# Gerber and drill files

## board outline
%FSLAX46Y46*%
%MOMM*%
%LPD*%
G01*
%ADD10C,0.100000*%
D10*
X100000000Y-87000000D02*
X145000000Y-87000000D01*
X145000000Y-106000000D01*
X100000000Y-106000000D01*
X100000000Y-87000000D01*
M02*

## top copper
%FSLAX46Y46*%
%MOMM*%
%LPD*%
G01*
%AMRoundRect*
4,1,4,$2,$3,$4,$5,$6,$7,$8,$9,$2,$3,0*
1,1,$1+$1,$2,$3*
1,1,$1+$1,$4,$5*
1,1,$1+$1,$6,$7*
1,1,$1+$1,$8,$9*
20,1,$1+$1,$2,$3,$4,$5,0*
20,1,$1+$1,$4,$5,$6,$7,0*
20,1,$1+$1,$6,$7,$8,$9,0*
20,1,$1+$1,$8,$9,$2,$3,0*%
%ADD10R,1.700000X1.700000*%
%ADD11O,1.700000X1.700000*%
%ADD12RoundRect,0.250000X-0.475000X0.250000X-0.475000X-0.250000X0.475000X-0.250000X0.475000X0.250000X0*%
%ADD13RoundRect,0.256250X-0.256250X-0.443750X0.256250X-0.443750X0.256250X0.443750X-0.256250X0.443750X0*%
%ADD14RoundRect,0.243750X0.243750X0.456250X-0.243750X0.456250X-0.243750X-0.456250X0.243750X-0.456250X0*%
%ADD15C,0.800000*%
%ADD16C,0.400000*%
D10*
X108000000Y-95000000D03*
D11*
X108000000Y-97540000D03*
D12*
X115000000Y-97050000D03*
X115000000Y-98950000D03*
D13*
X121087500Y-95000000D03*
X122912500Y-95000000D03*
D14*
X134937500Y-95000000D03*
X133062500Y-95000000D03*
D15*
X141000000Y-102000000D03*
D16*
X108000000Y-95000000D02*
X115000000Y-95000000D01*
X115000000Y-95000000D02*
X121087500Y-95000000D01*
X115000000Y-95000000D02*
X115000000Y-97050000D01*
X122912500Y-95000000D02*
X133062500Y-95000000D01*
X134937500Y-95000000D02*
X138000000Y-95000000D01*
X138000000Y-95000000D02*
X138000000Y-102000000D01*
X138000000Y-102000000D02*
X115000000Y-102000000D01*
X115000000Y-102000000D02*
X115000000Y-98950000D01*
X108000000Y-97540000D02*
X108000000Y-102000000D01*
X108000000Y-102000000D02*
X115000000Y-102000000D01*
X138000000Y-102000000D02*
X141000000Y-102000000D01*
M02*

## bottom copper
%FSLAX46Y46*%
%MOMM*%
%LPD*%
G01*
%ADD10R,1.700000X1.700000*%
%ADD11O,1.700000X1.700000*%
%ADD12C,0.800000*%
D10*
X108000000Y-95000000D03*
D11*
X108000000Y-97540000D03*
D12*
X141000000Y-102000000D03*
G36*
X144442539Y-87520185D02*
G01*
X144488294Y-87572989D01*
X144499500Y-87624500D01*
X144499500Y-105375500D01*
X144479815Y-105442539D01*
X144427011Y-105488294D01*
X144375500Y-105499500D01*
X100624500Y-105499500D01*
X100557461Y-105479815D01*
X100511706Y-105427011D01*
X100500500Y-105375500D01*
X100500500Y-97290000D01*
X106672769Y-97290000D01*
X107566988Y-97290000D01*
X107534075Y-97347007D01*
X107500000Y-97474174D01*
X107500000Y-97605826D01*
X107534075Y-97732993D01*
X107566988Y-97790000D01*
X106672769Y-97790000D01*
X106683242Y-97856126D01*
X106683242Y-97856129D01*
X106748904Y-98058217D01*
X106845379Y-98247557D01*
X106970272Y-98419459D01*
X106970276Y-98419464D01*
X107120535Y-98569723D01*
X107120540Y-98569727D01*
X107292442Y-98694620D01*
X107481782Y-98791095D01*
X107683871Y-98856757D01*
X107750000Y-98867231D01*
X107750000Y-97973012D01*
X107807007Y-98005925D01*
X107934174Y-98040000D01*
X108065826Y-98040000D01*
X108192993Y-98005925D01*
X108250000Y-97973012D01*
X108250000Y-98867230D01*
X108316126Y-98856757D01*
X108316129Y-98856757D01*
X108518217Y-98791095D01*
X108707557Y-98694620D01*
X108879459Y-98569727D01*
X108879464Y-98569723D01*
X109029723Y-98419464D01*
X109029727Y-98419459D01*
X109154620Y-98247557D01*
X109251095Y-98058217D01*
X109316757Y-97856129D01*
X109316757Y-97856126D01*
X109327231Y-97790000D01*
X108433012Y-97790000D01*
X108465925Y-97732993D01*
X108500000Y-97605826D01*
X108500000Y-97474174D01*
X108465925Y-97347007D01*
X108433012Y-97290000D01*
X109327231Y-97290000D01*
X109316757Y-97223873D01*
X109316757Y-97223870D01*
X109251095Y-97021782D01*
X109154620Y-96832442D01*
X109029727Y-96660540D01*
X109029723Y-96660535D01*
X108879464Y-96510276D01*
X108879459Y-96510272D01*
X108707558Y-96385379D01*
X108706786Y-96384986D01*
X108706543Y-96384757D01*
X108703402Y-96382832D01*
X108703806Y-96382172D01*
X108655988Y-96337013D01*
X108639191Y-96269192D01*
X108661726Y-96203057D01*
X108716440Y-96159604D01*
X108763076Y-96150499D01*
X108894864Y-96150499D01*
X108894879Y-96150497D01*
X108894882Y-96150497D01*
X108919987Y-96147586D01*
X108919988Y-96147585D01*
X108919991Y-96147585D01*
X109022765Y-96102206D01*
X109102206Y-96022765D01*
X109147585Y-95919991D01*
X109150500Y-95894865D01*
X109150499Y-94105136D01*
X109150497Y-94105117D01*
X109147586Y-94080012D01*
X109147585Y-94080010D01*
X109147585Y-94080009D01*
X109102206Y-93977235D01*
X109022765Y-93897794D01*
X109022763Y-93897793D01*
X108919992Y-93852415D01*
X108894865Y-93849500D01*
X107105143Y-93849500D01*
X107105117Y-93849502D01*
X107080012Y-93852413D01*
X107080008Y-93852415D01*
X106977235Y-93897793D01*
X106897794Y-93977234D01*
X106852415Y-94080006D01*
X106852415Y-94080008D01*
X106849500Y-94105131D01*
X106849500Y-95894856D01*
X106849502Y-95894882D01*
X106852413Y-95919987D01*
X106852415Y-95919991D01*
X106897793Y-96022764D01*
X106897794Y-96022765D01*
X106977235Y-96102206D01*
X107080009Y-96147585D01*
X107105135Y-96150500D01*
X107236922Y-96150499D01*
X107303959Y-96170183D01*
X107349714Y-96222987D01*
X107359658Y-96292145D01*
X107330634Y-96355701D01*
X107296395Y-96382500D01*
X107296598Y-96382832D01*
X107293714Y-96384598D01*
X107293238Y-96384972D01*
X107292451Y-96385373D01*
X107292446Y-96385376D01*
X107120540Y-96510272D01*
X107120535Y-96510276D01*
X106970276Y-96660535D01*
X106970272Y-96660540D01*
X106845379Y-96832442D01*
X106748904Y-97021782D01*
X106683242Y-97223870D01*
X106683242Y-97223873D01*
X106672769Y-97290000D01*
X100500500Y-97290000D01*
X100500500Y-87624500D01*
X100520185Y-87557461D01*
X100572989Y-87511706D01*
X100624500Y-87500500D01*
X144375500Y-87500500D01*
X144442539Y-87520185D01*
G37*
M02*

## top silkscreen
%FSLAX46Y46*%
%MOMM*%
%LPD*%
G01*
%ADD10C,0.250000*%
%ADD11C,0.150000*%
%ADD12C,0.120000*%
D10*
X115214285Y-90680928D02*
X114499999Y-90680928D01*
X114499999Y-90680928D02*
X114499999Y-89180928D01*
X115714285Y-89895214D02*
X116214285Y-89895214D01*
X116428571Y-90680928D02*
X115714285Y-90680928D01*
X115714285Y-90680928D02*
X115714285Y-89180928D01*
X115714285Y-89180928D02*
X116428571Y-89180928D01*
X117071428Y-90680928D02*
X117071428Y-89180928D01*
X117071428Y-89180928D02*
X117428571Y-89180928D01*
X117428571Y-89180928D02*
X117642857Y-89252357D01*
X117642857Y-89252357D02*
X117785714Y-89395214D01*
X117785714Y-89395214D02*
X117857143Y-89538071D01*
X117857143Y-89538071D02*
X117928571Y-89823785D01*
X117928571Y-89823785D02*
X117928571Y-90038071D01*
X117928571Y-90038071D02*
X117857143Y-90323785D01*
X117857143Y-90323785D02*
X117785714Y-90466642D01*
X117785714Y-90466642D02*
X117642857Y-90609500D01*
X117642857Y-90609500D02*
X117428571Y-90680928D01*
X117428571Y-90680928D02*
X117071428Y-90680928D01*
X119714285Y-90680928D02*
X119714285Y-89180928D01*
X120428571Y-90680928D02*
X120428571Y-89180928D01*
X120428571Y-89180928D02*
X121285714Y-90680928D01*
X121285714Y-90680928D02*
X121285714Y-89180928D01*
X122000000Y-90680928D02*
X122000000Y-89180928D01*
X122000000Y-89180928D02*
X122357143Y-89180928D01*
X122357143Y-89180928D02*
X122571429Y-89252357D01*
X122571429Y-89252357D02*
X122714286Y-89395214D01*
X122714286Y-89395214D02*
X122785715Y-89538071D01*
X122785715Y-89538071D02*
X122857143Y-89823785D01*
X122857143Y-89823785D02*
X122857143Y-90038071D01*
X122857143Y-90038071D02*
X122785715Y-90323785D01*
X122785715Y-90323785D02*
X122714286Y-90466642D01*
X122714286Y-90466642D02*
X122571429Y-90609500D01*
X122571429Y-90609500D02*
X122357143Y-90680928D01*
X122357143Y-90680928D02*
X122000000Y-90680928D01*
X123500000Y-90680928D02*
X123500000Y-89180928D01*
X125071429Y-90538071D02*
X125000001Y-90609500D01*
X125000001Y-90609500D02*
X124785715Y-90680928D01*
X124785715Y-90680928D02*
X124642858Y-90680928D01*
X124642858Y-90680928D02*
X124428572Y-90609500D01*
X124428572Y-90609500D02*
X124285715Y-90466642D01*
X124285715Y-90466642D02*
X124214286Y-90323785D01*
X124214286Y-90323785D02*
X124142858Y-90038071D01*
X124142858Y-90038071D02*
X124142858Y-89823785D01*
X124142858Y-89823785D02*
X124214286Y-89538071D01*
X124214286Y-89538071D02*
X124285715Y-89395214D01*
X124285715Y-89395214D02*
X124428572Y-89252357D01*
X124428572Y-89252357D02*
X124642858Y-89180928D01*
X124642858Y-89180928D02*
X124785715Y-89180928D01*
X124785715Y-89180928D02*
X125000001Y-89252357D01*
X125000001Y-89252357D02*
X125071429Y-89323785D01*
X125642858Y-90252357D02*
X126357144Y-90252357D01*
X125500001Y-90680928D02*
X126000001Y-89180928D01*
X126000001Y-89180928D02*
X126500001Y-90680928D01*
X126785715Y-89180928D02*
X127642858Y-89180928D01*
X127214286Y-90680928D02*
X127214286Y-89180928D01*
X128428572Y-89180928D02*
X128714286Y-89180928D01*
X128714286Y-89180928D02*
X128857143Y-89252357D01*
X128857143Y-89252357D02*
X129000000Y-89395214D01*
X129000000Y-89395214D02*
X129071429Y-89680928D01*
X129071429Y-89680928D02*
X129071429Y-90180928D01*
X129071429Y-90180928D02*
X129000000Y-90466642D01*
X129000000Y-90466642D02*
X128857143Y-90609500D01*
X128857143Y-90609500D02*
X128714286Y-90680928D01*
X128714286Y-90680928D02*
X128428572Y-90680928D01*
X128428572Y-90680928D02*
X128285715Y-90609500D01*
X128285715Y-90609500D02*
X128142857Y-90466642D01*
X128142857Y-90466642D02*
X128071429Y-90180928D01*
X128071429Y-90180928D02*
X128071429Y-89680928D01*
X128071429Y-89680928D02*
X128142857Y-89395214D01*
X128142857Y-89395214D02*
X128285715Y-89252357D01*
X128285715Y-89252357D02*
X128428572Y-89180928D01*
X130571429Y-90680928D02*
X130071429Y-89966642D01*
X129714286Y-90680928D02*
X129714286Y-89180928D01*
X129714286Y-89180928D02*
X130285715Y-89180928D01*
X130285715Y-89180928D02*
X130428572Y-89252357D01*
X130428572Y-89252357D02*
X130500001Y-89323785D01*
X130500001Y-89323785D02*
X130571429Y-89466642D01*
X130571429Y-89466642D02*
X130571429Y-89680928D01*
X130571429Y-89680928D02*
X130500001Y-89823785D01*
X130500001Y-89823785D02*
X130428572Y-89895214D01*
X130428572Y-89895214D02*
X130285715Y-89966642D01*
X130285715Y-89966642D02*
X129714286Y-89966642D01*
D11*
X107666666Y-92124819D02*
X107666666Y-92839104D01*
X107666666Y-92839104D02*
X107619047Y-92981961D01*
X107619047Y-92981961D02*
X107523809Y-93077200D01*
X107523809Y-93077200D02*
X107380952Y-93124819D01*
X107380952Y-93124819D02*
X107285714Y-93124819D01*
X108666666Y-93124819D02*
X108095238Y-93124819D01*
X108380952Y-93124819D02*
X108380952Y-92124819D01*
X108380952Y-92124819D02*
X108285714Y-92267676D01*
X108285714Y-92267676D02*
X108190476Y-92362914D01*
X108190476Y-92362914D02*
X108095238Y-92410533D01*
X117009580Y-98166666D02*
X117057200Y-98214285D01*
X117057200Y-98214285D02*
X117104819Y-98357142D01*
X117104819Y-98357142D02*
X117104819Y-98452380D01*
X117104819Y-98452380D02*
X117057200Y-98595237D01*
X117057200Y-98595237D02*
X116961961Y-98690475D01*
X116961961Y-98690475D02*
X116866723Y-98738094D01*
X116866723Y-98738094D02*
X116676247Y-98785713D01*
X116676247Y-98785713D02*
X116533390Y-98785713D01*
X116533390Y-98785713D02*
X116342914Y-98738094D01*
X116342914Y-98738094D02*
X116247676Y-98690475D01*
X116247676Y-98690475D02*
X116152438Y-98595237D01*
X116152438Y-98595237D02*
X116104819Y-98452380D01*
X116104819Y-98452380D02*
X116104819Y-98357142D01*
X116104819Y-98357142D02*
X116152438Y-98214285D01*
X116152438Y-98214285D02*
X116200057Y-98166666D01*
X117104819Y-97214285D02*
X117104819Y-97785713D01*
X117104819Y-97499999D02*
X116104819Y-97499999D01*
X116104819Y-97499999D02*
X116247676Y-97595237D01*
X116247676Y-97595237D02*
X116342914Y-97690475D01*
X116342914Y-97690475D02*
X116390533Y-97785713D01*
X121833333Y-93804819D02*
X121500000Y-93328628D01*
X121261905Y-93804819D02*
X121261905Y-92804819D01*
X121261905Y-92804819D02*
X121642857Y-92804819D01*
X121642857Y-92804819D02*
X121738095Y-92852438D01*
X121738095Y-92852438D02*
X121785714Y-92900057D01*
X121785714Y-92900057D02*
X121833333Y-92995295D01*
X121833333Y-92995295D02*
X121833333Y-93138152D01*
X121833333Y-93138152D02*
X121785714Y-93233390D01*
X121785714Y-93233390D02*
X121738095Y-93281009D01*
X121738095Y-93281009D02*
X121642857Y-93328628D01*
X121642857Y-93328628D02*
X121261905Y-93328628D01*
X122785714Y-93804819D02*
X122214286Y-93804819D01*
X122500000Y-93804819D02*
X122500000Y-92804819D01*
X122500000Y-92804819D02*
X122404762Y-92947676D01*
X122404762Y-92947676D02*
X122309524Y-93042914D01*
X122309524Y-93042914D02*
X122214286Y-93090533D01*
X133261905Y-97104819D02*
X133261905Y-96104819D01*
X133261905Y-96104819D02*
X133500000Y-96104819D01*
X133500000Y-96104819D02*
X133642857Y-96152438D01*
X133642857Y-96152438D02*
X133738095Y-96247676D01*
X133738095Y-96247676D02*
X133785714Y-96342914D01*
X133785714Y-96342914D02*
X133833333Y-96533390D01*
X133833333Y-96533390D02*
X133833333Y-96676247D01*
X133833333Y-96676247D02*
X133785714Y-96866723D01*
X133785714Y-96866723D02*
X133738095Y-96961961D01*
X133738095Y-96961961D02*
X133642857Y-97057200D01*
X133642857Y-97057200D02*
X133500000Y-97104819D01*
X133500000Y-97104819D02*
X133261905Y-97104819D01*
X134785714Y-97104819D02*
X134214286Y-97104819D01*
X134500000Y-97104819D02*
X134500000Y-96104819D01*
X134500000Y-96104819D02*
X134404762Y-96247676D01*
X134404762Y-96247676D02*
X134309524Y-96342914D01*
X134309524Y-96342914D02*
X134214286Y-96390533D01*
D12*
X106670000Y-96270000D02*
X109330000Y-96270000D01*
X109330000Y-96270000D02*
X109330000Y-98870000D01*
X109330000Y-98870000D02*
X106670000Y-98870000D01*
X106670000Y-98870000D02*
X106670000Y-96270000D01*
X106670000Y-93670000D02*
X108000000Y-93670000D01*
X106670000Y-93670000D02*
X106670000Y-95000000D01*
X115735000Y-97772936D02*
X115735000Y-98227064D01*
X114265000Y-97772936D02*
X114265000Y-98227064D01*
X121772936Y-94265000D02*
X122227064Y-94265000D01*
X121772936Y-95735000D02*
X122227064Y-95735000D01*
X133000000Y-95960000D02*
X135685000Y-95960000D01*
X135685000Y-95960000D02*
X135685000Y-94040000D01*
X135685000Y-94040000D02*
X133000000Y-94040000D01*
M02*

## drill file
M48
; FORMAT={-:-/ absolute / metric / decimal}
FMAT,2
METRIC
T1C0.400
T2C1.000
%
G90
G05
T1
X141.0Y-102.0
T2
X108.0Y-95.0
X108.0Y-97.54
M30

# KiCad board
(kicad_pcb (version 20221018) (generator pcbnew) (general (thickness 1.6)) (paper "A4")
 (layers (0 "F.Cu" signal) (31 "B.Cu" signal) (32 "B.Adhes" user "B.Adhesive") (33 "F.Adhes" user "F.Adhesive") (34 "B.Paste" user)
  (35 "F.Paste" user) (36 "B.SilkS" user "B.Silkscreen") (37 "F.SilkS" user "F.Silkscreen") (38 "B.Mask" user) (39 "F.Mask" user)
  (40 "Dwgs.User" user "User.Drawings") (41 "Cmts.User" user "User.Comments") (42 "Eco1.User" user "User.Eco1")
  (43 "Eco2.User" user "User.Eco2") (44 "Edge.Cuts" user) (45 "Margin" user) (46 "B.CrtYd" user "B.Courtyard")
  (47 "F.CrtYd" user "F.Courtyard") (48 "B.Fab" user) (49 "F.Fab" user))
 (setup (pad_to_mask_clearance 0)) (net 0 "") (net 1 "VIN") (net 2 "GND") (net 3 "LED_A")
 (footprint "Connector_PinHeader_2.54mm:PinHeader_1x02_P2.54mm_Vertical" (layer "F.Cu") (at 108 95)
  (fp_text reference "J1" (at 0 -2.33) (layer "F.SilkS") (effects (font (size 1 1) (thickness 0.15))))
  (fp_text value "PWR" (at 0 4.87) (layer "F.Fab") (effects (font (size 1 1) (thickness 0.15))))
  (fp_line (start -1.33 1.27) (end 1.33 1.27) (stroke (width 0.12) (type solid)) (layer "F.SilkS"))
  (fp_line (start 1.33 1.27) (end 1.33 3.87) (stroke (width 0.12) (type solid)) (layer "F.SilkS"))
  (fp_line (start 1.33 3.87) (end -1.33 3.87) (stroke (width 0.12) (type solid)) (layer "F.SilkS"))
  (fp_line (start -1.33 3.87) (end -1.33 1.27) (stroke (width 0.12) (type solid)) (layer "F.SilkS"))
  (fp_line (start -1.33 -1.33) (end 0 -1.33) (stroke (width 0.12) (type solid)) (layer "F.SilkS"))
  (fp_line (start -1.33 -1.33) (end -1.33 0) (stroke (width 0.12) (type solid)) (layer "F.SilkS"))
  (pad "1" thru_hole rect (at 0 0) (size 1.7 1.7) (drill 1) (layers "*.Cu" "*.Mask") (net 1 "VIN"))
  (pad "2" thru_hole oval (at 0 2.54) (size 1.7 1.7) (drill 1) (layers "*.Cu" "*.Mask") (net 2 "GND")))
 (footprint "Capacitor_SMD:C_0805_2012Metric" (layer "F.Cu") (at 115 98 270)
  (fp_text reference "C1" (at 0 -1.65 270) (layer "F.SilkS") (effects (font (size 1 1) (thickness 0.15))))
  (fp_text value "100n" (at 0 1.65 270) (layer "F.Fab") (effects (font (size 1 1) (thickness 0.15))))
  (fp_line (start -0.227064 -0.735) (end 0.227064 -0.735) (stroke (width 0.12) (type solid)) (layer "F.SilkS"))
  (fp_line (start -0.227064 0.735) (end 0.227064 0.735) (stroke (width 0.12) (type solid)) (layer "F.SilkS"))
  (pad "1" smd roundrect (at -0.95 0 270) (size 1 1.45) (layers "F.Cu" "F.Paste" "F.Mask") (roundrect_rratio 0.25) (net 1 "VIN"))
  (pad "2" smd roundrect (at 0.95 0 270) (size 1 1.45) (layers "F.Cu" "F.Paste" "F.Mask") (roundrect_rratio 0.25) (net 2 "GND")))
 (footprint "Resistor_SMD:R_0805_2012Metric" (layer "F.Cu") (at 122 95)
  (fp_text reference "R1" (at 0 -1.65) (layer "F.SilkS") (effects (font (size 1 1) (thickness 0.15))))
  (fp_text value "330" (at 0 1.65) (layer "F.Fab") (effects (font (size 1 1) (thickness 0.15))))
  (fp_line (start -0.227064 -0.735) (end 0.227064 -0.735) (stroke (width 0.12) (type solid)) (layer "F.SilkS"))
  (fp_line (start -0.227064 0.735) (end 0.227064 0.735) (stroke (width 0.12) (type solid)) (layer "F.SilkS"))
  (pad "1" smd roundrect (at -0.9125 0) (size 1.025 1.4) (layers "F.Cu" "F.Paste" "F.Mask") (roundrect_rratio 0.25) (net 1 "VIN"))
  (pad "2" smd roundrect (at 0.9125 0) (size 1.025 1.4) (layers "F.Cu" "F.Paste" "F.Mask") (roundrect_rratio 0.25) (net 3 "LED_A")))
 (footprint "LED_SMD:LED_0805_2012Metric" (layer "F.Cu") (at 134 95 180)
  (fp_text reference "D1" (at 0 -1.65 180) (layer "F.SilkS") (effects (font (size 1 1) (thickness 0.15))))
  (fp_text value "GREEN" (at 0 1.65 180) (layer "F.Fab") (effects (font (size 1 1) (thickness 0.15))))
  (fp_line (start 1 -0.96) (end -1.685 -0.96) (stroke (width 0.12) (type solid)) (layer "F.SilkS"))
  (fp_line (start -1.685 -0.96) (end -1.685 0.96) (stroke (width 0.12) (type solid)) (layer "F.SilkS"))
  (fp_line (start -1.685 0.96) (end 1 0.96) (stroke (width 0.12) (type solid)) (layer "F.SilkS"))
  (pad "1" smd roundrect (at -0.9375 0 180) (size 0.975 1.4) (layers "F.Cu" "F.Paste" "F.Mask") (roundrect_rratio 0.25) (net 2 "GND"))
  (pad "2" smd roundrect (at 0.9375 0 180) (size 0.975 1.4) (layers "F.Cu" "F.Paste" "F.Mask") (roundrect_rratio 0.25) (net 3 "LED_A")))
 (gr_rect (start 100 87) (end 145 106) (stroke (width 0.1) (type default)) (fill none) (layer "Edge.Cuts"))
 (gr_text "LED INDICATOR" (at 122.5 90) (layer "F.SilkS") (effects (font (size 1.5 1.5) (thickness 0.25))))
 (segment (start 108 95) (end 115 95) (width 0.4) (layer "F.Cu") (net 1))
 (segment (start 115 95) (end 121.0875 95) (width 0.4) (layer "F.Cu") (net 1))
 (segment (start 115 95) (end 115 97.05) (width 0.4) (layer "F.Cu") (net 1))
 (segment (start 122.9125 95) (end 133.0625 95) (width 0.4) (layer "F.Cu") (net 3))
 (segment (start 134.9375 95) (end 138 95) (width 0.4) (layer "F.Cu") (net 2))
 (segment (start 138 95) (end 138 102) (width 0.4) (layer "F.Cu") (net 2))
 (segment (start 138 102) (end 115 102) (width 0.4) (layer "F.Cu") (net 2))
 (segment (start 115 102) (end 115 98.95) (width 0.4) (layer "F.Cu") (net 2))
 (segment (start 108 97.54) (end 108 102) (width 0.4) (layer "F.Cu") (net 2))
 (segment (start 108 102) (end 115 102) (width 0.4) (layer "F.Cu") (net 2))
 (segment (start 138 102) (end 141 102) (width 0.4) (layer "F.Cu") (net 2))
 (via (at 141 102) (size 0.8) (drill 0.4) (layers "F.Cu" "B.Cu") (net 2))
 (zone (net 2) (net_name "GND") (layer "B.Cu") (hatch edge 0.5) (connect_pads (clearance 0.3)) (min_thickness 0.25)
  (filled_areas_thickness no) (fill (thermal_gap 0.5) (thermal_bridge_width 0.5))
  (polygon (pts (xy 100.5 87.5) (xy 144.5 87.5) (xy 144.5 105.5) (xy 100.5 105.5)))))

